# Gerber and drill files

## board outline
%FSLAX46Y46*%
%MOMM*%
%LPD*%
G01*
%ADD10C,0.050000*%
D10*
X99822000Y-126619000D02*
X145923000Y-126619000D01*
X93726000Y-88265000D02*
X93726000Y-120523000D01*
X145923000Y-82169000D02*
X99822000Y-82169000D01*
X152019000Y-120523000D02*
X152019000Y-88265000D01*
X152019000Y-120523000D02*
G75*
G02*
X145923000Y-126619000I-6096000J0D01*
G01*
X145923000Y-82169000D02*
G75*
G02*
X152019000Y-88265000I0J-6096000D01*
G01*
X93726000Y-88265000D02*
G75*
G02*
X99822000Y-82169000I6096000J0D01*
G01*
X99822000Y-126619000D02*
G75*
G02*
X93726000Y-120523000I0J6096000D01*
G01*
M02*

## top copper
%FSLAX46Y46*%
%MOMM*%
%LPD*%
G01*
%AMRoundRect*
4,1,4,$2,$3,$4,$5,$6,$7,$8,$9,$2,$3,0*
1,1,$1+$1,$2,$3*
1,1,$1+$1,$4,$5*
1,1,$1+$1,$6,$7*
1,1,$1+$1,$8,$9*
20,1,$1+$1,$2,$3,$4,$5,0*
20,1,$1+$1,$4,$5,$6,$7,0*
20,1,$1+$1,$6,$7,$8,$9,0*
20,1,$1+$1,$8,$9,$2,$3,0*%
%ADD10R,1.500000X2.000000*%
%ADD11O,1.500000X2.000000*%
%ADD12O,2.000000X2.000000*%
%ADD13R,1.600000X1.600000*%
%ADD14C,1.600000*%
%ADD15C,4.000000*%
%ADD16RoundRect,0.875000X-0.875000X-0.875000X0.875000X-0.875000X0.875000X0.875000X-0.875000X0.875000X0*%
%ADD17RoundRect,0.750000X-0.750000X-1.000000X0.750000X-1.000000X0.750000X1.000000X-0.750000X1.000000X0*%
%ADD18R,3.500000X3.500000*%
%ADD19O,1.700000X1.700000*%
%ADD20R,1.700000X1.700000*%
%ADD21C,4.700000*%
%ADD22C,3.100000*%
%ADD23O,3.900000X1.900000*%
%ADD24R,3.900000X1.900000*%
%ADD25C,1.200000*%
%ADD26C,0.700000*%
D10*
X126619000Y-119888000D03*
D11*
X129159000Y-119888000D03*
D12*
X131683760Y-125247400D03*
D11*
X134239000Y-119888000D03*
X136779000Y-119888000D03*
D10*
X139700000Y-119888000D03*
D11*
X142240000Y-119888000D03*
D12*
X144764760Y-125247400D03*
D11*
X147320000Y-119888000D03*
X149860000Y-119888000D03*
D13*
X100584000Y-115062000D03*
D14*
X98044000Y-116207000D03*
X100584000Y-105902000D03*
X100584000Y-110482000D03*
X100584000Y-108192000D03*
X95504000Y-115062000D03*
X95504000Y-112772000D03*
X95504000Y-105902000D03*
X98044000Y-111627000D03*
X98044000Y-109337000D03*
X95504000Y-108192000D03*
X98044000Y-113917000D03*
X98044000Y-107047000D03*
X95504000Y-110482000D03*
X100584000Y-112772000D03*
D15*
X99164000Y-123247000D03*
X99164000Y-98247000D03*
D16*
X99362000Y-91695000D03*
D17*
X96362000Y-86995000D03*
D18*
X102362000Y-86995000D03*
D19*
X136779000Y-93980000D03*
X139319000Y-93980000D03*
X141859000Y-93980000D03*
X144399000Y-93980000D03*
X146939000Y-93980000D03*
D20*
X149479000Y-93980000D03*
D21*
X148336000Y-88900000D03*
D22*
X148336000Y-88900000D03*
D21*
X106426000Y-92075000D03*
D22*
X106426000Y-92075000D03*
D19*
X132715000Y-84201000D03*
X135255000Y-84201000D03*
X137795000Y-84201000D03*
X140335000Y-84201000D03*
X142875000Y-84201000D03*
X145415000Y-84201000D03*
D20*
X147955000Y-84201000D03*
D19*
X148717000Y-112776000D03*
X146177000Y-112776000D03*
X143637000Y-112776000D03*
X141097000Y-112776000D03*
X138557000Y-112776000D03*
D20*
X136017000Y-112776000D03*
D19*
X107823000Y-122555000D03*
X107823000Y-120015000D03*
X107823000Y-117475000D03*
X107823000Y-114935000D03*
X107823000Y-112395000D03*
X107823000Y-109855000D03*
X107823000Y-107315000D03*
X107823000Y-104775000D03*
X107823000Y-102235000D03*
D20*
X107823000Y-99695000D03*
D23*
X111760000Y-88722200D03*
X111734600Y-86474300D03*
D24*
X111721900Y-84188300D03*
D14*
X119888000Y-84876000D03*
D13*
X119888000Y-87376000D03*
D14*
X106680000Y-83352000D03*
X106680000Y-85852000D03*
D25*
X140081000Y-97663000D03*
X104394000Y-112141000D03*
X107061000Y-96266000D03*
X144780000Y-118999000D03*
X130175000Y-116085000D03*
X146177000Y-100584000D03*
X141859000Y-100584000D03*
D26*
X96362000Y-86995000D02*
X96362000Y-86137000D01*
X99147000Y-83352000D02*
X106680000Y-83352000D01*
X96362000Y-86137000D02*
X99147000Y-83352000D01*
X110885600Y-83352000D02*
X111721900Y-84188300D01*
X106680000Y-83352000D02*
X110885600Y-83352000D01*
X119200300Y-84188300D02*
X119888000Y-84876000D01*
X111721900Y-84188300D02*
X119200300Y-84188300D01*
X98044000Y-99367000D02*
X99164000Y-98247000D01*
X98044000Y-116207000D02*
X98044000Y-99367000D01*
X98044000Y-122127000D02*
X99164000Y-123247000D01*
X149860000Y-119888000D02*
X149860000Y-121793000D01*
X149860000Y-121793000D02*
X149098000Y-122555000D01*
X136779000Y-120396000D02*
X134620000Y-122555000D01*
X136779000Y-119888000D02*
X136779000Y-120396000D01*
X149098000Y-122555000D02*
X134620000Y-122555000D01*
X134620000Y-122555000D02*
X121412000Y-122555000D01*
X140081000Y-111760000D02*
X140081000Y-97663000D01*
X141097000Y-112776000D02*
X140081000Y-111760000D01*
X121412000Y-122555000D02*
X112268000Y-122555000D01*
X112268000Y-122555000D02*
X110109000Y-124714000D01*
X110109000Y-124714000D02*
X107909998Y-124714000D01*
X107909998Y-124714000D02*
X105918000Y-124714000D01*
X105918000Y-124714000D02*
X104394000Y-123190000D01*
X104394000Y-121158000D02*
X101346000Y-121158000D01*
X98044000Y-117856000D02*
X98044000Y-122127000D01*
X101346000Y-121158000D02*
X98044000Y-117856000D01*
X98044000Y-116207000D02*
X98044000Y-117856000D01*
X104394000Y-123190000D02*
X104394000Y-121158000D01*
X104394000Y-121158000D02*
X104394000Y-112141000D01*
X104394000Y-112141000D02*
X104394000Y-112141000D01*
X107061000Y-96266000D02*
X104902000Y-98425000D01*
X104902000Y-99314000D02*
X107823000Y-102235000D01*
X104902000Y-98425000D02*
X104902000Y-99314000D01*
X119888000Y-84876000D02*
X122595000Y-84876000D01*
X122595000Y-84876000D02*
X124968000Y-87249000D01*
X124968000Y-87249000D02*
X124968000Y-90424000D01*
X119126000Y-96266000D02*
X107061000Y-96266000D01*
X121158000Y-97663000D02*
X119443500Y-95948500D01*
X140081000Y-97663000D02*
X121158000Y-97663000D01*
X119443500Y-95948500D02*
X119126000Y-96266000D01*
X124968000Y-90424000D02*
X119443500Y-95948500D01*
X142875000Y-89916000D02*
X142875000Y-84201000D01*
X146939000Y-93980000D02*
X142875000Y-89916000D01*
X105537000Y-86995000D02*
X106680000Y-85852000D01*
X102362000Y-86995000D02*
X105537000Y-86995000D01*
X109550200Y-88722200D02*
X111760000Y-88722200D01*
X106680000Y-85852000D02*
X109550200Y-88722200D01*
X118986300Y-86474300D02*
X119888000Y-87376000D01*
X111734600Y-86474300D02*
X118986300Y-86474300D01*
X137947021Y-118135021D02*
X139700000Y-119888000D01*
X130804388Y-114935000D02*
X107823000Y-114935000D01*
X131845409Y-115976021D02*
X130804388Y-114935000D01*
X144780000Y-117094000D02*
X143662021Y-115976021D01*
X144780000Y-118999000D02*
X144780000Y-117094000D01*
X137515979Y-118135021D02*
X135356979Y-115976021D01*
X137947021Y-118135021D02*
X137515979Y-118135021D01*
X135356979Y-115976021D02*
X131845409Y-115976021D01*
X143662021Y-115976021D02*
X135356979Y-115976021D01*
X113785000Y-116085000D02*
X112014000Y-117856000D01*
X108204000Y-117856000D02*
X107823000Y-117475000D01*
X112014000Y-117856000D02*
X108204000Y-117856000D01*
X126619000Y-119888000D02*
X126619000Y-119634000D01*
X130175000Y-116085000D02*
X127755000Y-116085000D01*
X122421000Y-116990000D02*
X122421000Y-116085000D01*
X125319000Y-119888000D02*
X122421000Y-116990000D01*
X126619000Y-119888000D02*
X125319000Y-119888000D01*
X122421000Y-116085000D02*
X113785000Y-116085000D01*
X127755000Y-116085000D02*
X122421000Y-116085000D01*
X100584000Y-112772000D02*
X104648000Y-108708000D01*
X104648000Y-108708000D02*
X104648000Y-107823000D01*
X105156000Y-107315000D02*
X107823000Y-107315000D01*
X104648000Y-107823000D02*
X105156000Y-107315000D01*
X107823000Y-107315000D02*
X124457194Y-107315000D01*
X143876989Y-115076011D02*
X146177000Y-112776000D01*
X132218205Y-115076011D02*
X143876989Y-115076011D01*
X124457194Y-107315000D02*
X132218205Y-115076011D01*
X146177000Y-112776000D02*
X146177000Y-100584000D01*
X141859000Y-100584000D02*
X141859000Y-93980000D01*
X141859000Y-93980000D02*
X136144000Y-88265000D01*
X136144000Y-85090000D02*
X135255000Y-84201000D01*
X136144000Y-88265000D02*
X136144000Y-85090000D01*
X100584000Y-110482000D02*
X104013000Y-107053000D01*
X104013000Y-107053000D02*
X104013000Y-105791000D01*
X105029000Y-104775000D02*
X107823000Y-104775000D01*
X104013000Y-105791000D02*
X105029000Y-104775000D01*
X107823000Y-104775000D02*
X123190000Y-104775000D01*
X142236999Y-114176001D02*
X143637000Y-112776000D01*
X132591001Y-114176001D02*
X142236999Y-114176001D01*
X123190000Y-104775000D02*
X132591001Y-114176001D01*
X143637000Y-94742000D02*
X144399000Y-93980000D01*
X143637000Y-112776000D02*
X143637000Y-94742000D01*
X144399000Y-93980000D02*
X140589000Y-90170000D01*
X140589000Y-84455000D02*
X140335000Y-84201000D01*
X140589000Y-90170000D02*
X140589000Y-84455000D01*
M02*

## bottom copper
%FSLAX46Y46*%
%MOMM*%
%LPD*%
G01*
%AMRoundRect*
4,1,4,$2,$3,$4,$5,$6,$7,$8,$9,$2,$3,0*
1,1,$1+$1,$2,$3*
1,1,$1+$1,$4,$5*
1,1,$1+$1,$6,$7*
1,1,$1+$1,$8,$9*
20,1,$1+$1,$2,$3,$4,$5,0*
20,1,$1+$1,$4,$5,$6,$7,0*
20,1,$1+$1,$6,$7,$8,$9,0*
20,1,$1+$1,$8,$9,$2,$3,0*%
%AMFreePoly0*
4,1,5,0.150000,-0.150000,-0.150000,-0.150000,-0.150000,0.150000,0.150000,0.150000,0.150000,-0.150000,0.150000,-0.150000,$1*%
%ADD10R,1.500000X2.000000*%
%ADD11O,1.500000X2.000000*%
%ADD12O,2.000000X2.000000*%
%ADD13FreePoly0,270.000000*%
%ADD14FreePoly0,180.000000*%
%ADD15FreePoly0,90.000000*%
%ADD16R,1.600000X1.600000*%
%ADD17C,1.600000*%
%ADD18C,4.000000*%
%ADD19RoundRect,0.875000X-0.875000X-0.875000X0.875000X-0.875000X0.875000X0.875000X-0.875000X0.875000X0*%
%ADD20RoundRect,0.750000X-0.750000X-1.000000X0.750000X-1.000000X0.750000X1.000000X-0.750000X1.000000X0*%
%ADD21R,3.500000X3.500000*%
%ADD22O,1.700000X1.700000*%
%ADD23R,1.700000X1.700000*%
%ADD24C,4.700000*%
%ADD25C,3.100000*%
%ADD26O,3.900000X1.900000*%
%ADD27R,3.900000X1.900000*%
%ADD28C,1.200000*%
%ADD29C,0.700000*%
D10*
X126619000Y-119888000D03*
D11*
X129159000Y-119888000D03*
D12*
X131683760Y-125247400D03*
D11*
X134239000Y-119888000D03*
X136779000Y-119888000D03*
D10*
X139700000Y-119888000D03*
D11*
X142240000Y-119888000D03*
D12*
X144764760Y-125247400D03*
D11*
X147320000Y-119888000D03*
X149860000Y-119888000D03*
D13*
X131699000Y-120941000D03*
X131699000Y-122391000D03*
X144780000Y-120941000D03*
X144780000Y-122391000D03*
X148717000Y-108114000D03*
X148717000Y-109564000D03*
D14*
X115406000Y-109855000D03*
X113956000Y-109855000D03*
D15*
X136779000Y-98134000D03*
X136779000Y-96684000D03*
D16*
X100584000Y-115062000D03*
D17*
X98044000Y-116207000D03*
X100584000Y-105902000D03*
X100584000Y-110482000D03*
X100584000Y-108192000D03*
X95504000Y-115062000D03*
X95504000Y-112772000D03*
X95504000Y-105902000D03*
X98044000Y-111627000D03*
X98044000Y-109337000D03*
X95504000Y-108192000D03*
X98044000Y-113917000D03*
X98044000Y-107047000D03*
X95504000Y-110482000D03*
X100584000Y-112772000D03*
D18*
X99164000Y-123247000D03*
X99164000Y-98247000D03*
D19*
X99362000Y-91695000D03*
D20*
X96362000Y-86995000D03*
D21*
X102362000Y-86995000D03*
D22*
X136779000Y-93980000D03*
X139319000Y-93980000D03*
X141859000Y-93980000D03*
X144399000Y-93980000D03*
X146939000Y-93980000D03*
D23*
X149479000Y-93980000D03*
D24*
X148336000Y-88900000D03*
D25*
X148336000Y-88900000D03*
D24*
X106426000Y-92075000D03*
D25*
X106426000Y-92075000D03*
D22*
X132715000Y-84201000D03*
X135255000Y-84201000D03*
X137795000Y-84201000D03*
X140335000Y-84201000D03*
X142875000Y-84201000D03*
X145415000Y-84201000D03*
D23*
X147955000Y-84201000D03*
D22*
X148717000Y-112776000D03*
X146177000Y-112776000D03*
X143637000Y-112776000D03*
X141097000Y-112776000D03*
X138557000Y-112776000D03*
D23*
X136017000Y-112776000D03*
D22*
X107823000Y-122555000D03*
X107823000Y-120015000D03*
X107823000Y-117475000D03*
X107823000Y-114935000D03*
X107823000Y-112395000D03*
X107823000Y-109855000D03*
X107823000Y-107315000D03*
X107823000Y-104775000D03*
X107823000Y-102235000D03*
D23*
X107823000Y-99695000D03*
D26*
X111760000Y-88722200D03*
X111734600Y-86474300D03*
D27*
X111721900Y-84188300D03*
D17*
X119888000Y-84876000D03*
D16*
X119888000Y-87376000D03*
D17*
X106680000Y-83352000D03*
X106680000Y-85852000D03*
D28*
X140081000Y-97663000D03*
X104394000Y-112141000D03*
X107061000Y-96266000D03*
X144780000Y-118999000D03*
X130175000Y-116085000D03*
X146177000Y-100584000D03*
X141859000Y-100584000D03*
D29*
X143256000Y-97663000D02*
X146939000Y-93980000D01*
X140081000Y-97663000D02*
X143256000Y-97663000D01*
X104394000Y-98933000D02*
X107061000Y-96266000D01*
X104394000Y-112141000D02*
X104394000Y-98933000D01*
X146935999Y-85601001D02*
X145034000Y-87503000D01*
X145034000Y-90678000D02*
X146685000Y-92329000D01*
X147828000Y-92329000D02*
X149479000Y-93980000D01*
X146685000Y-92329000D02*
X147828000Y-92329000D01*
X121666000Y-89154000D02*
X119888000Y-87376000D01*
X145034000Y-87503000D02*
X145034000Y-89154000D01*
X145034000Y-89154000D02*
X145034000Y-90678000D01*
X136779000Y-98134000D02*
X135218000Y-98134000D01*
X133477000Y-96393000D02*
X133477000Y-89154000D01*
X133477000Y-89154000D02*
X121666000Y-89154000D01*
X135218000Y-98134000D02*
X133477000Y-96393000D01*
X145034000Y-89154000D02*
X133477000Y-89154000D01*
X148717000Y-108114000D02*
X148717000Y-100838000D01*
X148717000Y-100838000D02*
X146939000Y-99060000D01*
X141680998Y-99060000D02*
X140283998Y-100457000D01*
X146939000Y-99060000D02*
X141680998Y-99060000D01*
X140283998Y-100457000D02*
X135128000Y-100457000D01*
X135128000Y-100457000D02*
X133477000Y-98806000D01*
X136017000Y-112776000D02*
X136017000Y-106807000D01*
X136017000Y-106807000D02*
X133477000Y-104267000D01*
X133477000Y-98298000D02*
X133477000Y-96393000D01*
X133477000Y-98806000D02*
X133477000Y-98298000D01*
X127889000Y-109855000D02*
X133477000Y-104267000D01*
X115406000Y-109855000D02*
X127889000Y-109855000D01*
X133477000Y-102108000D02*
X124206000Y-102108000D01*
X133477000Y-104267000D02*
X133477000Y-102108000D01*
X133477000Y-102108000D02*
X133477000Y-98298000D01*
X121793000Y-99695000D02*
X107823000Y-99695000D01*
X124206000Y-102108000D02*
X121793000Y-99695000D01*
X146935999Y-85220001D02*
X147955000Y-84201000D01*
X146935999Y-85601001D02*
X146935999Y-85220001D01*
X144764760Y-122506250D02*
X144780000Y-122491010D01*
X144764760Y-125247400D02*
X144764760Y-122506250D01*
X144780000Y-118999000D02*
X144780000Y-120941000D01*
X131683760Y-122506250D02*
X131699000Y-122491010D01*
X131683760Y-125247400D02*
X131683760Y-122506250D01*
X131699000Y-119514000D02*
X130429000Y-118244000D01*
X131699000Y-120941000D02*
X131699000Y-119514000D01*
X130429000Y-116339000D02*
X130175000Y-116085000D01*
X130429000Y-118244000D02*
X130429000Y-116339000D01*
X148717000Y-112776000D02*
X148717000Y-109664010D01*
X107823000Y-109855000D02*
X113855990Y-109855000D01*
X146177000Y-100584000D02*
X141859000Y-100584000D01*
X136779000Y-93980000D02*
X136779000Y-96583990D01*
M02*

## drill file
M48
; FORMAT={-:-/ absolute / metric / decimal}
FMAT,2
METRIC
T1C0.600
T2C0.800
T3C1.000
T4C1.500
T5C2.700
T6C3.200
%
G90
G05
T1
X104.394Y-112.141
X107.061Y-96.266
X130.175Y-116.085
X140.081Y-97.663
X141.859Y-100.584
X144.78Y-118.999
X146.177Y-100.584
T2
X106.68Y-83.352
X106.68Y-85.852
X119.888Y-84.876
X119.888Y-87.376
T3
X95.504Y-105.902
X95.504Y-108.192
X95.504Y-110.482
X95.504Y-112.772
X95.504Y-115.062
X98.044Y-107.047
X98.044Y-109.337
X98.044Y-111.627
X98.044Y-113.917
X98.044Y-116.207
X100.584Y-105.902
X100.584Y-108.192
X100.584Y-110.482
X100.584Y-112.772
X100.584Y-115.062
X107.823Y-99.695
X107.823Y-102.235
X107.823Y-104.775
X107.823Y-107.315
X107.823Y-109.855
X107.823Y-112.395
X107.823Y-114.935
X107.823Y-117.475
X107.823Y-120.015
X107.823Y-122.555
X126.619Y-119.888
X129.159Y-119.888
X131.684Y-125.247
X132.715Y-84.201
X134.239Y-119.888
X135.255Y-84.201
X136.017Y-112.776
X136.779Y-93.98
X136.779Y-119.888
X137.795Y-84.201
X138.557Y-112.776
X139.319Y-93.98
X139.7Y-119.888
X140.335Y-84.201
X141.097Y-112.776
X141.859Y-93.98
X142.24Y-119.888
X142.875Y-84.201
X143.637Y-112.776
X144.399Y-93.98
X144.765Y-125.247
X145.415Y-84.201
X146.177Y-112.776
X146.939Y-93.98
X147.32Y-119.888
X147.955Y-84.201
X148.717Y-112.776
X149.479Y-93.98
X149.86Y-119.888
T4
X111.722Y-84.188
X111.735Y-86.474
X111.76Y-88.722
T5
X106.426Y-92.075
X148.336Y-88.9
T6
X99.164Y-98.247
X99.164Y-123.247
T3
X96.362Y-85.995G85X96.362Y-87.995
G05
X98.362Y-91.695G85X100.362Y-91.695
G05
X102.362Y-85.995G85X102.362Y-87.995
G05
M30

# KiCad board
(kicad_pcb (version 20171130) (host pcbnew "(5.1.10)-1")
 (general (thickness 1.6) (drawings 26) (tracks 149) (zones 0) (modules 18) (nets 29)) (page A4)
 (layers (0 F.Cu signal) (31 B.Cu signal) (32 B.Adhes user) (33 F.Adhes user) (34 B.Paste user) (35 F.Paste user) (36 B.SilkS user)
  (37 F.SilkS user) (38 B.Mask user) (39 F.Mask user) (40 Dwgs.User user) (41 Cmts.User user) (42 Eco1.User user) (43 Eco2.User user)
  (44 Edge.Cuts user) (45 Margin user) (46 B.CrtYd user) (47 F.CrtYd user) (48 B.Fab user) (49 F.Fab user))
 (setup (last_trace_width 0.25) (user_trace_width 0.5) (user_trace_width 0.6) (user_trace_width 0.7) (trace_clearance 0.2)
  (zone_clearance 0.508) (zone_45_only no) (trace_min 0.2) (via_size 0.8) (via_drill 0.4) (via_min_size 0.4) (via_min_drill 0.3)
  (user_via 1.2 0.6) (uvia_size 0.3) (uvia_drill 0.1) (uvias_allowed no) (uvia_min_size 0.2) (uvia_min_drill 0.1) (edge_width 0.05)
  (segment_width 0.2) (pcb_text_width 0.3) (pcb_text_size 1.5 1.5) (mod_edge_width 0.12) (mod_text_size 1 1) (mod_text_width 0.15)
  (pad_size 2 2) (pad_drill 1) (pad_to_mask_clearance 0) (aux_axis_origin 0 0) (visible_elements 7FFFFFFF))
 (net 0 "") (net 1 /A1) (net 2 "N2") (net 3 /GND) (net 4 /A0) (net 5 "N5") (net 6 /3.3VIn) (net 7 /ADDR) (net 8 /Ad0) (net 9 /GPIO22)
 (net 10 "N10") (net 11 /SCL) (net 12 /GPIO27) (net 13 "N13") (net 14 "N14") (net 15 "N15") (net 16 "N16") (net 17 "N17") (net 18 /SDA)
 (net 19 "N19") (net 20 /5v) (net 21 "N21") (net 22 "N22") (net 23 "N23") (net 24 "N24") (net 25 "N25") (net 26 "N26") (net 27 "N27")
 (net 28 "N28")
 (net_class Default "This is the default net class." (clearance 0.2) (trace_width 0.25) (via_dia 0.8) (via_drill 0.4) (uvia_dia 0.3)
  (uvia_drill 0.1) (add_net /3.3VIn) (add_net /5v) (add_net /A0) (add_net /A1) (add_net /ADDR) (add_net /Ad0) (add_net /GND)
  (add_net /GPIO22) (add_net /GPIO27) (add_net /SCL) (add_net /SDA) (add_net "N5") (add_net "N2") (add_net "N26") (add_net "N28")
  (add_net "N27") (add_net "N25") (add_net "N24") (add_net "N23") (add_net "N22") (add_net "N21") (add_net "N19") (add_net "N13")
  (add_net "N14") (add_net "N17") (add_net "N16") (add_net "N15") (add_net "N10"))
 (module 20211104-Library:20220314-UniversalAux (layer F.Cu) (at 131.699 121.158 180)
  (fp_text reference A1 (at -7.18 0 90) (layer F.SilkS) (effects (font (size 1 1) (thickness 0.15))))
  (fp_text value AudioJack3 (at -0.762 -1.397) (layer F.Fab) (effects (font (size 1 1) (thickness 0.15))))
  (pad S thru_hole rect (at 5.08 1.27 180) (size 1.5 2) (drill 1) (layers *.Cu *.Mask) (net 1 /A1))
  (pad "" thru_hole oval (at 2.54 1.27 180) (size 1.5 2) (drill 1) (layers *.Cu *.Mask))
  (pad R thru_hole oval (at 0.01524 -4.0894 180) (size 2 2) (drill 1) (layers *.Cu *.Mask) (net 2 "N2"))
  (pad "" thru_hole oval (at -2.54 1.27 180) (size 1.5 2) (drill 1) (layers *.Cu *.Mask))
  (pad T thru_hole oval (at -5.08 1.27 180) (size 1.5 2) (drill 1) (layers *.Cu *.Mask) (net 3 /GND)))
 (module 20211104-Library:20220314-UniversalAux (layer F.Cu) (at 144.78 121.158 180)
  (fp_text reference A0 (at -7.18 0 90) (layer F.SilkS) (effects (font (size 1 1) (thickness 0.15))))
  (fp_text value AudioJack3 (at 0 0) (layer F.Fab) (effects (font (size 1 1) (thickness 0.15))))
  (pad S thru_hole rect (at 5.08 1.27 180) (size 1.5 2) (drill 1) (layers *.Cu *.Mask) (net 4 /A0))
  (pad "" thru_hole oval (at 2.54 1.27 180) (size 1.5 2) (drill 1) (layers *.Cu *.Mask))
  (pad R thru_hole oval (at 0.01524 -4.0894 180) (size 2 2) (drill 1) (layers *.Cu *.Mask) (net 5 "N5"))
  (pad "" thru_hole oval (at -2.54 1.27 180) (size 1.5 2) (drill 1) (layers *.Cu *.Mask))
  (pad T thru_hole oval (at -5.08 1.27 180) (size 1.5 2) (drill 1) (layers *.Cu *.Mask) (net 3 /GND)))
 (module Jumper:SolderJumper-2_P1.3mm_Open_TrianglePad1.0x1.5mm (layer B.Cu) (at 131.699 121.666 270)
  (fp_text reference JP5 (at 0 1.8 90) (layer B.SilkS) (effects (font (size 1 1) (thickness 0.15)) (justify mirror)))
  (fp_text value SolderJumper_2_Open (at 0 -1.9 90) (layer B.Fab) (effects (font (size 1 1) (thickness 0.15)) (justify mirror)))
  (pad 1 smd custom (at -0.725 0 270) (size 0.3 0.3) (layers B.Cu B.Mask) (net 1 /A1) (zone_connect 2)
   (options (clearance outline) (anchor rect)) (primitives))
  (pad 2 smd custom (at 0.725 0 270) (size 0.3 0.3) (layers B.Cu B.Mask) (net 2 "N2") (zone_connect 2)
   (options (clearance outline) (anchor rect)) (primitives)))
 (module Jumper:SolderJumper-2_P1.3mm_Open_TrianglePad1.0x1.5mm (layer B.Cu) (at 144.78 121.666 270)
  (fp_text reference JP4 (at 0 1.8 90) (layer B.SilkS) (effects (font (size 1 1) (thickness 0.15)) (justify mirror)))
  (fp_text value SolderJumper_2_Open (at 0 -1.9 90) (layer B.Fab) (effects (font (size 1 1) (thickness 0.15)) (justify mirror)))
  (pad 1 smd custom (at -0.725 0 270) (size 0.3 0.3) (layers B.Cu B.Mask) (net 4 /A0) (zone_connect 2)
   (options (clearance outline) (anchor rect)) (primitives))
  (pad 2 smd custom (at 0.725 0 270) (size 0.3 0.3) (layers B.Cu B.Mask) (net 5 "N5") (zone_connect 2)
   (options (clearance outline) (anchor rect)) (primitives)))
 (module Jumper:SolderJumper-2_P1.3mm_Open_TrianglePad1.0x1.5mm (layer B.Cu) (at 148.717 108.839 270)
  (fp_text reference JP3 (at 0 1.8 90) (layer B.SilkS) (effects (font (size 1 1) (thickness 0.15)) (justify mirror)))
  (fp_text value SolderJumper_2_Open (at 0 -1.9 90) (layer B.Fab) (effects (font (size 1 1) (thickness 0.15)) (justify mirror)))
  (pad 1 smd custom (at -0.725 0 270) (size 0.3 0.3) (layers B.Cu B.Mask) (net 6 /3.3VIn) (zone_connect 2)
   (options (clearance outline) (anchor rect)) (primitives))
  (pad 2 smd custom (at 0.725 0 270) (size 0.3 0.3) (layers B.Cu B.Mask) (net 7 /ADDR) (zone_connect 2)
   (options (clearance outline) (anchor rect)) (primitives)))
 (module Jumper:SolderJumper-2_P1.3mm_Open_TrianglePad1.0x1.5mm (layer B.Cu) (at 114.681 109.855 180)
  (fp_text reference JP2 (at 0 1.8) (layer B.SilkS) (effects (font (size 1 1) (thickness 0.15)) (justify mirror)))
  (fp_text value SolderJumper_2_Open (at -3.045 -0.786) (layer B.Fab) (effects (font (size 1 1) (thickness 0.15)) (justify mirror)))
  (pad 1 smd custom (at -0.725 0 180) (size 0.3 0.3) (layers B.Cu B.Mask) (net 6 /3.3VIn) (zone_connect 2)
   (options (clearance outline) (anchor rect)) (primitives))
  (pad 2 smd custom (at 0.725 0 180) (size 0.3 0.3) (layers B.Cu B.Mask) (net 7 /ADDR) (zone_connect 2)
   (options (clearance outline) (anchor rect)) (primitives)))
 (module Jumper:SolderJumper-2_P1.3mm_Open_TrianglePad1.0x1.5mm (layer B.Cu) (at 136.779 97.409 90)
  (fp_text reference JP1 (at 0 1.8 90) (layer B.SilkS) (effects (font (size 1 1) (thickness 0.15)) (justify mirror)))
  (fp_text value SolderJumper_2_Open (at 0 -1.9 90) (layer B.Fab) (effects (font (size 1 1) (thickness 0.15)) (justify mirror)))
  (pad 1 smd custom (at -0.725 0 90) (size 0.3 0.3) (layers B.Cu B.Mask) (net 6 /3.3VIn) (zone_connect 2)
   (options (clearance outline) (anchor rect)) (primitives))
  (pad 2 smd custom (at 0.725 0 90) (size 0.3 0.3) (layers B.Cu B.Mask) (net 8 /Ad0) (zone_connect 2)
   (options (clearance outline) (anchor rect)) (primitives)))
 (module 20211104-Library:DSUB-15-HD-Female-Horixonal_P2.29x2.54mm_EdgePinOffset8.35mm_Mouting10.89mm (layer F.Cu) (at 100.584 115.062 270)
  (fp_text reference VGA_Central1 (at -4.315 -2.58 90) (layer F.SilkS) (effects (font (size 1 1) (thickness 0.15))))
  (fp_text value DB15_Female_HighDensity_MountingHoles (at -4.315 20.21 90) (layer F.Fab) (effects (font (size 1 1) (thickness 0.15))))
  (pad 1 thru_hole rect (at 0 0 270) (size 1.6 1.6) (drill 1) (layers *.Cu *.Mask) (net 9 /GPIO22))
  (pad 6 thru_hole circle (at 1.145 2.54 270) (size 1.6 1.6) (drill 1) (layers *.Cu *.Mask) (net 3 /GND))
  (pad 5 thru_hole circle (at -9.16 0 270) (size 1.6 1.6) (drill 1) (layers *.Cu *.Mask) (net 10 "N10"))
  (pad 3 thru_hole circle (at -4.58 0 270) (size 1.6 1.6) (drill 1) (layers *.Cu *.Mask) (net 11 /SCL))
  (pad 4 thru_hole circle (at -6.87 0 270) (size 1.6 1.6) (drill 1) (layers *.Cu *.Mask) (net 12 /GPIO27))
  (pad 11 thru_hole circle (at 0 5.08 270) (size 1.6 1.6) (drill 1) (layers *.Cu *.Mask) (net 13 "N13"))
  (pad 12 thru_hole circle (at -2.29 5.08 270) (size 1.6 1.6) (drill 1) (layers *.Cu *.Mask) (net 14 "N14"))
  (pad 15 thru_hole circle (at -9.16 5.08 270) (size 1.6 1.6) (drill 1) (layers *.Cu *.Mask) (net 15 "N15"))
  (pad 8 thru_hole circle (at -3.435 2.54 270) (size 1.6 1.6) (drill 1) (layers *.Cu *.Mask) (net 3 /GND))
  (pad 9 thru_hole circle (at -5.725 2.54 270) (size 1.6 1.6) (drill 1) (layers *.Cu *.Mask) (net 3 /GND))
  (pad 14 thru_hole circle (at -6.87 5.08 270) (size 1.6 1.6) (drill 1) (layers *.Cu *.Mask) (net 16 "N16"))
  (pad 7 thru_hole circle (at -1.145 2.54 270) (size 1.6 1.6) (drill 1) (layers *.Cu *.Mask) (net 3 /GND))
  (pad 10 thru_hole circle (at -8.015 2.54 270) (size 1.6 1.6) (drill 1) (layers *.Cu *.Mask) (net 3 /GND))
  (pad 13 thru_hole circle (at -4.58 5.08 270) (size 1.6 1.6) (drill 1) (layers *.Cu *.Mask) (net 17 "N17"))
  (pad 2 thru_hole circle (at -2.29 0 270) (size 1.6 1.6) (drill 1) (layers *.Cu *.Mask) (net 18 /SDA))
  (pad 0 thru_hole circle (at 8.185 1.42 270) (size 4 4) (drill 3.2) (layers *.Cu *.Mask) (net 3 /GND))
  (pad 0 thru_hole circle (at -16.815 1.42 270) (size 4 4) (drill 3.2) (layers *.Cu *.Mask) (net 3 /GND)))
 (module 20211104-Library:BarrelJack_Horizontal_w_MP (layer F.Cu) (at 102.362 86.995)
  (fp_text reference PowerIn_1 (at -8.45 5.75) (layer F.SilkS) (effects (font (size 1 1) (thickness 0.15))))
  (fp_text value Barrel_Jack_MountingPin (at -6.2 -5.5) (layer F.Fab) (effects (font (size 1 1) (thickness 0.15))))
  (pad MP thru_hole roundrect (at -3 4.7) (size 3.5 3.5) (drill oval 3 1) (layers *.Cu *.Mask) (roundrect_rratio 0.25) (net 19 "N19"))
  (pad 2 thru_hole roundrect (at -6 0) (size 3 3.5) (drill oval 1 3) (layers *.Cu *.Mask) (roundrect_rratio 0.25) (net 3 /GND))
  (pad 1 thru_hole rect (at 0 0) (size 3.5 3.5) (drill oval 1 3) (layers *.Cu *.Mask) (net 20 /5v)))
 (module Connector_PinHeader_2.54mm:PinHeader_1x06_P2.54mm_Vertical (layer F.Cu) (at 149.479 93.98 270)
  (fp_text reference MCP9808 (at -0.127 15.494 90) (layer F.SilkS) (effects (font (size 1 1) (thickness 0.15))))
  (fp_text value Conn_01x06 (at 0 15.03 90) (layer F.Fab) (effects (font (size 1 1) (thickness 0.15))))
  (pad 6 thru_hole oval (at 0 12.7 270) (size 1.7 1.7) (drill 1) (layers *.Cu *.Mask) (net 8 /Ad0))
  (pad 5 thru_hole oval (at 0 10.16 270) (size 1.7 1.7) (drill 1) (layers *.Cu *.Mask) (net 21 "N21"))
  (pad 4 thru_hole oval (at 0 7.62 270) (size 1.7 1.7) (drill 1) (layers *.Cu *.Mask) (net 18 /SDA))
  (pad 3 thru_hole oval (at 0 5.08 270) (size 1.7 1.7) (drill 1) (layers *.Cu *.Mask) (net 11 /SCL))
  (pad 2 thru_hole oval (at 0 2.54 270) (size 1.7 1.7) (drill 1) (layers *.Cu *.Mask) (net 3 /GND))
  (pad 1 thru_hole rect (at 0 0 270) (size 1.7 1.7) (drill 1) (layers *.Cu *.Mask) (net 6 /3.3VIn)))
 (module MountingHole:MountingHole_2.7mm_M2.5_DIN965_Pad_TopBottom (layer F.Cu) (at 148.336 88.9)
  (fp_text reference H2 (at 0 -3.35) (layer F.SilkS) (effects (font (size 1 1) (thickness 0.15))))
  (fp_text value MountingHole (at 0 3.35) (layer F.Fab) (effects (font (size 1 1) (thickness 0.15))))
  (pad 1 connect circle (at 0 0) (size 4.7 4.7) (layers B.Cu B.Mask))
  (pad 1 connect circle (at 0 0) (size 4.7 4.7) (layers F.Cu F.Mask))
  (pad 1 thru_hole circle (at 0 0) (size 3.1 3.1) (drill 2.7) (layers *.Cu *.Mask)))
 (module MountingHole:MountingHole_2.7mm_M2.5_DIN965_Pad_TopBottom (layer F.Cu) (at 106.426 92.075)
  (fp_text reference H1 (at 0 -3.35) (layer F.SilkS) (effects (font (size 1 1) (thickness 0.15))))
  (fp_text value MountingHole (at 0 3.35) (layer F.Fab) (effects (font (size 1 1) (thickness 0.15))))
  (pad 1 connect circle (at 0 0) (size 4.7 4.7) (layers B.Cu B.Mask))
  (pad 1 connect circle (at 0 0) (size 4.7 4.7) (layers F.Cu F.Mask))
  (pad 1 thru_hole circle (at 0 0) (size 3.1 3.1) (drill 2.7) (layers *.Cu *.Mask)))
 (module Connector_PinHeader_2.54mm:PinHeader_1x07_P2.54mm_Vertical (layer F.Cu) (at 147.955 84.201 270)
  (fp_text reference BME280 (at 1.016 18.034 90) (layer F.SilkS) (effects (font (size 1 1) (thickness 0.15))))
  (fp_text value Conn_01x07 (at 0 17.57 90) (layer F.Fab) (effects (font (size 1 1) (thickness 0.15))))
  (pad 7 thru_hole oval (at 0 15.24 270) (size 1.7 1.7) (drill 1) (layers *.Cu *.Mask) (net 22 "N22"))
  (pad 6 thru_hole oval (at 0 12.7 270) (size 1.7 1.7) (drill 1) (layers *.Cu *.Mask) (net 18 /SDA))
  (pad 5 thru_hole oval (at 0 10.16 270) (size 1.7 1.7) (drill 1) (layers *.Cu *.Mask) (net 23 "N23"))
  (pad 4 thru_hole oval (at 0 7.62 270) (size 1.7 1.7) (drill 1) (layers *.Cu *.Mask) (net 11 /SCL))
  (pad 3 thru_hole oval (at 0 5.08 270) (size 1.7 1.7) (drill 1) (layers *.Cu *.Mask) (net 3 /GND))
  (pad 2 thru_hole oval (at 0 2.54 270) (size 1.7 1.7) (drill 1) (layers *.Cu *.Mask) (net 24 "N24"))
  (pad 1 thru_hole rect (at 0 0 270) (size 1.7 1.7) (drill 1) (layers *.Cu *.Mask) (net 6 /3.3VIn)))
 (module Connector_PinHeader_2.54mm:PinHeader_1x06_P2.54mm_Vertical (layer F.Cu) (at 136.017 112.776 90)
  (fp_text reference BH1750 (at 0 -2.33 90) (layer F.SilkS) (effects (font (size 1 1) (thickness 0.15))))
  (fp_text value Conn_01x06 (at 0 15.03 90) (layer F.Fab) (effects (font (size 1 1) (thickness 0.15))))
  (pad 6 thru_hole oval (at 0 12.7 90) (size 1.7 1.7) (drill 1) (layers *.Cu *.Mask) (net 7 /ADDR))
  (pad 5 thru_hole oval (at 0 10.16 90) (size 1.7 1.7) (drill 1) (layers *.Cu *.Mask) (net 18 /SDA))
  (pad 4 thru_hole oval (at 0 7.62 90) (size 1.7 1.7) (drill 1) (layers *.Cu *.Mask) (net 11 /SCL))
  (pad 3 thru_hole oval (at 0 5.08 90) (size 1.7 1.7) (drill 1) (layers *.Cu *.Mask) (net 3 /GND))
  (pad 2 thru_hole oval (at 0 2.54 90) (size 1.7 1.7) (drill 1) (layers *.Cu *.Mask) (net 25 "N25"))
  (pad 1 thru_hole rect (at 0 0 90) (size 1.7 1.7) (drill 1) (layers *.Cu *.Mask) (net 6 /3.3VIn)))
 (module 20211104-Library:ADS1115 (layer F.Cu) (at 107.823 99.695)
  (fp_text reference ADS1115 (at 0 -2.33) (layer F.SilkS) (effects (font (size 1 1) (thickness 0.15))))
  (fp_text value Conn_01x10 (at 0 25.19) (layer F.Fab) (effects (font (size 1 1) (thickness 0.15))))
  (pad 10 thru_hole oval (at 0 22.86) (size 1.7 1.7) (drill 1) (layers *.Cu *.Mask) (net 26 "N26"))
  (pad 9 thru_hole oval (at 0 20.32) (size 1.7 1.7) (drill 1) (layers *.Cu *.Mask) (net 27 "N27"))
  (pad 8 thru_hole oval (at 0 17.78) (size 1.7 1.7) (drill 1) (layers *.Cu *.Mask) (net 1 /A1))
  (pad 7 thru_hole oval (at 0 15.24) (size 1.7 1.7) (drill 1) (layers *.Cu *.Mask) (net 4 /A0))
  (pad 6 thru_hole oval (at 0 12.7) (size 1.7 1.7) (drill 1) (layers *.Cu *.Mask) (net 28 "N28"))
  (pad 5 thru_hole oval (at 0 10.16) (size 1.7 1.7) (drill 1) (layers *.Cu *.Mask) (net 7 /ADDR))
  (pad 4 thru_hole oval (at 0 7.62) (size 1.7 1.7) (drill 1) (layers *.Cu *.Mask) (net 18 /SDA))
  (pad 3 thru_hole oval (at 0 5.08) (size 1.7 1.7) (drill 1) (layers *.Cu *.Mask) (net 11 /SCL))
  (pad 2 thru_hole oval (at 0 2.54) (size 1.7 1.7) (drill 1) (layers *.Cu *.Mask) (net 3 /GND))
  (pad 1 thru_hole rect (at 0 0) (size 1.7 1.7) (drill 1) (layers *.Cu *.Mask) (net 6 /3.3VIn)))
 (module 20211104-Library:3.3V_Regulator (layer F.Cu) (at 111.76 81.026 270)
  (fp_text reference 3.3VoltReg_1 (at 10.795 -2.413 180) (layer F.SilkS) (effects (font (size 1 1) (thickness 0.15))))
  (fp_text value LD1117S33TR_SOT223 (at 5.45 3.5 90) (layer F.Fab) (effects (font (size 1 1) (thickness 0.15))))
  (pad 3 thru_hole oval (at 7.6962 0 270) (size 1.9 3.9) (drill 1.5) (layers *.Cu *.Mask) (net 20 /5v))
  (pad 2 thru_hole oval (at 5.4483 0.0254 270) (size 1.9 3.9) (drill 1.5) (layers *.Cu *.Mask) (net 6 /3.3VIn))
  (pad 1 thru_hole rect (at 3.1623 0.0381 270) (size 1.9 3.9) (drill 1.5) (layers *.Cu *.Mask) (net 3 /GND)))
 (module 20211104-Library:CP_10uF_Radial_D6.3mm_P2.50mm (layer F.Cu) (at 119.888 87.376 90)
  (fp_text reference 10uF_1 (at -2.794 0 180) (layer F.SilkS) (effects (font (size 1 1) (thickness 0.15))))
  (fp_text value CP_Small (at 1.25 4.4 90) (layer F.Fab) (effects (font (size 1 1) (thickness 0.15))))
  (pad 2 thru_hole circle (at 2.5 0 90) (size 1.6 1.6) (drill 0.8) (layers *.Cu *.Mask) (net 3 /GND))
  (pad 1 thru_hole rect (at 0 0 90) (size 1.6 1.6) (drill 0.8) (layers *.Cu *.Mask) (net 6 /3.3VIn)))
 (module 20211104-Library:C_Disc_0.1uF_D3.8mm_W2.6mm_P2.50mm (layer F.Cu) (at 106.68 85.852 90)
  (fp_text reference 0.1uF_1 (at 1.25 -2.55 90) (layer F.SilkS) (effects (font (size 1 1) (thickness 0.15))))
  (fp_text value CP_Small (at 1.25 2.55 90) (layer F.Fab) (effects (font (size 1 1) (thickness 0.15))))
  (pad 2 thru_hole circle (at 2.5 0 90) (size 1.6 1.6) (drill 0.8) (layers *.Cu *.Mask) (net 3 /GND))
  (pad 1 thru_hole circle (at 0 0 90) (size 1.6 1.6) (drill 0.8) (layers *.Cu *.Mask) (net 20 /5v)))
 (gr_line (start 99.822 126.619) (end 145.923 126.619) (layer Edge.Cuts) (width 0.05))
 (gr_line (start 93.726 88.265) (end 93.726 120.523) (layer Edge.Cuts) (width 0.05))
 (gr_line (start 145.923 82.169) (end 99.822 82.169) (layer Edge.Cuts) (width 0.05))
 (gr_line (start 152.019 120.523) (end 152.019 88.265) (layer Edge.Cuts) (width 0.05))
 (gr_arc (start 145.923 120.523) (end 145.923 126.619) (angle -90) (layer Edge.Cuts) (width 0.05))
 (gr_arc (start 145.923 88.265) (end 152.019 88.265) (angle -90) (layer Edge.Cuts) (width 0.05))
 (gr_arc (start 99.822 88.265) (end 99.822 82.169) (angle -90) (layer Edge.Cuts) (width 0.05))
 (gr_arc (start 99.822 120.523) (end 93.726 120.523) (angle -90) (layer Edge.Cuts) (width 0.05))
 (segment (start 96.362 86.995) (end 96.362 86.137) (width 0.7) (layer F.Cu) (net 3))
 (segment (start 99.147 83.352) (end 106.68 83.352) (width 0.7) (layer F.Cu) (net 3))
 (segment (start 96.362 86.137) (end 99.147 83.352) (width 0.7) (layer F.Cu) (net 3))
 (segment (start 110.8856 83.352) (end 111.7219 84.1883) (width 0.7) (layer F.Cu) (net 3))
 (segment (start 106.68 83.352) (end 110.8856 83.352) (width 0.7) (layer F.Cu) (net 3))
 (segment (start 119.2003 84.1883) (end 119.888 84.876) (width 0.7) (layer F.Cu) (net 3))
 (segment (start 111.7219 84.1883) (end 119.2003 84.1883) (width 0.7) (layer F.Cu) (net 3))
 (segment (start 98.044 99.367) (end 99.164 98.247) (width 0.7) (layer F.Cu) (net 3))
 (segment (start 98.044 116.207) (end 98.044 99.367) (width 0.7) (layer F.Cu) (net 3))
 (segment (start 98.044 122.127) (end 99.164 123.247) (width 0.7) (layer F.Cu) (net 3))
 (segment (start 149.86 119.888) (end 149.86 121.793) (width 0.7) (layer F.Cu) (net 3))
 (segment (start 149.86 121.793) (end 149.098 122.555) (width 0.7) (layer F.Cu) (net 3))
 (segment (start 136.779 120.396) (end 134.62 122.555) (width 0.7) (layer F.Cu) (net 3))
 (segment (start 136.779 119.888) (end 136.779 120.396) (width 0.7) (layer F.Cu) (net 3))
 (segment (start 149.098 122.555) (end 134.62 122.555) (width 0.7) (layer F.Cu) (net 3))
 (segment (start 134.62 122.555) (end 121.412 122.555) (width 0.7) (layer F.Cu) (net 3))
 (via (at 140.081 97.663) (size 1.2) (drill 0.6) (layers F.Cu B.Cu) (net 3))
 (segment (start 140.081 111.76) (end 140.081 97.663) (width 0.7) (layer F.Cu) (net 3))
 (segment (start 141.097 112.776) (end 140.081 111.76) (width 0.7) (layer F.Cu) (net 3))
 (segment (start 143.256 97.663) (end 146.939 93.98) (width 0.7) (layer B.Cu) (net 3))
 (segment (start 140.081 97.663) (end 143.256 97.663) (width 0.7) (layer B.Cu) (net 3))
 (segment (start 121.412 122.555) (end 112.268 122.555) (width 0.7) (layer F.Cu) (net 3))
 (segment (start 112.268 122.555) (end 110.109 124.714) (width 0.7) (layer F.Cu) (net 3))
 (segment (start 110.109 124.714) (end 107.909998 124.714) (width 0.7) (layer F.Cu) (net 3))
 (segment (start 107.909998 124.714) (end 105.918 124.714) (width 0.7) (layer F.Cu) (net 3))
 (segment (start 105.918 124.714) (end 104.394 123.19) (width 0.7) (layer F.Cu) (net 3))
 (segment (start 104.394 121.158) (end 101.346 121.158) (width 0.7) (layer F.Cu) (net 3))
 (segment (start 98.044 117.856) (end 98.044 122.127) (width 0.7) (layer F.Cu) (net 3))
 (segment (start 101.346 121.158) (end 98.044 117.856) (width 0.7) (layer F.Cu) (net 3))
 (segment (start 98.044 116.207) (end 98.044 117.856) (width 0.7) (layer F.Cu) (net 3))
 (segment (start 104.394 123.19) (end 104.394 121.158) (width 0.7) (layer F.Cu) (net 3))
 (segment (start 104.394 121.158) (end 104.394 112.141) (width 0.7) (layer F.Cu) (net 3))
 (segment (start 104.394 112.141) (end 104.394 112.141) (width 0.7) (layer F.Cu) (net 3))
 (via (at 104.394 112.141) (size 1.2) (drill 0.6) (layers F.Cu B.Cu) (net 3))
 (via (at 107.061 96.266) (size 1.2) (drill 0.6) (layers F.Cu B.Cu) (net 3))
 (segment (start 104.394 98.933) (end 107.061 96.266) (width 0.7) (layer B.Cu) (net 3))
 (segment (start 104.394 112.141) (end 104.394 98.933) (width 0.7) (layer B.Cu) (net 3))
 (segment (start 107.061 96.266) (end 104.902 98.425) (width 0.7) (layer F.Cu) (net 3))
 (segment (start 104.902 99.314) (end 107.823 102.235) (width 0.7) (layer F.Cu) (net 3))
 (segment (start 104.902 98.425) (end 104.902 99.314) (width 0.7) (layer F.Cu) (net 3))
 (segment (start 119.888 84.876) (end 122.595 84.876) (width 0.7) (layer F.Cu) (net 3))
 (segment (start 122.595 84.876) (end 124.968 87.249) (width 0.7) (layer F.Cu) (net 3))
 (segment (start 124.968 87.249) (end 124.968 90.424) (width 0.7) (layer F.Cu) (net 3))
 (segment (start 119.126 96.266) (end 107.061 96.266) (width 0.7) (layer F.Cu) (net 3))
 (segment (start 121.158 97.663) (end 119.4435 95.9485) (width 0.7) (layer F.Cu) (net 3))
 (segment (start 140.081 97.663) (end 121.158 97.663) (width 0.7) (layer F.Cu) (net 3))
 (segment (start 119.4435 95.9485) (end 119.126 96.266) (width 0.7) (layer F.Cu) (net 3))
 (segment (start 124.968 90.424) (end 119.4435 95.9485) (width 0.7) (layer F.Cu) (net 3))
 (segment (start 142.875 89.916) (end 142.875 84.201) (width 0.7) (layer F.Cu) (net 3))
 (segment (start 146.939 93.98) (end 142.875 89.916) (width 0.7) (layer F.Cu) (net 3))
 (segment (start 105.537 86.995) (end 106.68 85.852) (width 0.7) (layer F.Cu) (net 20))
 (segment (start 102.362 86.995) (end 105.537 86.995) (width 0.7) (layer F.Cu) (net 20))
 (segment (start 109.5502 88.7222) (end 111.76 88.7222) (width 0.7) (layer F.Cu) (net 20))
 (segment (start 106.68 85.852) (end 109.5502 88.7222) (width 0.7) (layer F.Cu) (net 20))
 (segment (start 118.9863 86.4743) (end 119.888 87.376) (width 0.7) (layer F.Cu) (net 6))
 (segment (start 111.7346 86.4743) (end 118.9863 86.4743) (width 0.7) (layer F.Cu) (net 6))
 (segment (start 146.935999 85.601001) (end 145.034 87.503) (width 0.7) (layer B.Cu) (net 6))
 (segment (start 145.034 90.678) (end 146.685 92.329) (width 0.7) (layer B.Cu) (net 6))
 (segment (start 147.828 92.329) (end 149.479 93.98) (width 0.7) (layer B.Cu) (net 6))
 (segment (start 146.685 92.329) (end 147.828 92.329) (width 0.7) (layer B.Cu) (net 6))
 (segment (start 121.666 89.154) (end 119.888 87.376) (width 0.7) (layer B.Cu) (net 6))
 (segment (start 145.034 87.503) (end 145.034 89.154) (width 0.7) (layer B.Cu) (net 6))
 (segment (start 145.034 89.154) (end 145.034 90.678) (width 0.7) (layer B.Cu) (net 6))
 (segment (start 136.779 98.134) (end 135.218 98.134) (width 0.7) (layer B.Cu) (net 6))
 (segment (start 133.477 96.393) (end 133.477 89.154) (width 0.7) (layer B.Cu) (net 6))
 (segment (start 133.477 89.154) (end 121.666 89.154) (width 0.7) (layer B.Cu) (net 6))
 (segment (start 135.218 98.134) (end 133.477 96.393) (width 0.7) (layer B.Cu) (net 6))
 (segment (start 145.034 89.154) (end 133.477 89.154) (width 0.7) (layer B.Cu) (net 6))
 (segment (start 148.717 108.114) (end 148.717 100.838) (width 0.7) (layer B.Cu) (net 6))
 (segment (start 148.717 100.838) (end 146.939 99.06) (width 0.7) (layer B.Cu) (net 6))
 (segment (start 141.680998 99.06) (end 140.283998 100.457) (width 0.7) (layer B.Cu) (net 6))
 (segment (start 146.939 99.06) (end 141.680998 99.06) (width 0.7) (layer B.Cu) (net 6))
 (segment (start 140.283998 100.457) (end 135.128 100.457) (width 0.7) (layer B.Cu) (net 6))
 (segment (start 135.128 100.457) (end 133.477 98.806) (width 0.7) (layer B.Cu) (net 6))
 (segment (start 136.017 112.776) (end 136.017 106.807) (width 0.7) (layer B.Cu) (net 6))
 (segment (start 136.017 106.807) (end 133.477 104.267) (width 0.7) (layer B.Cu) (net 6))
 (segment (start 133.477 98.298) (end 133.477 96.393) (width 0.7) (layer B.Cu) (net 6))
 (segment (start 133.477 98.806) (end 133.477 98.298) (width 0.7) (layer B.Cu) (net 6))
 (segment (start 127.889 109.855) (end 133.477 104.267) (width 0.7) (layer B.Cu) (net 6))
 (segment (start 115.406 109.855) (end 127.889 109.855) (width 0.7) (layer B.Cu) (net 6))
 (segment (start 133.477 102.108) (end 124.206 102.108) (width 0.7) (layer B.Cu) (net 6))
 (segment (start 133.477 104.267) (end 133.477 102.108) (width 0.7) (layer B.Cu) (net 6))
 (segment (start 133.477 102.108) (end 133.477 98.298) (width 0.7) (layer B.Cu) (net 6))
 (segment (start 121.793 99.695) (end 107.823 99.695) (width 0.7) (layer B.Cu) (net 6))
 (segment (start 124.206 102.108) (end 121.793 99.695) (width 0.7) (layer B.Cu) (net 6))
 (segment (start 146.935999 85.220001) (end 147.955 84.201) (width 0.7) (layer B.Cu) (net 6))
 (segment (start 146.935999 85.601001) (end 146.935999 85.220001) (width 0.7) (layer B.Cu) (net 6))
 (segment (start 144.76476 122.50625) (end 144.78 122.49101) (width 0.7) (layer B.Cu) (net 5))
 (segment (start 144.76476 125.2474) (end 144.76476 122.50625) (width 0.7) (layer B.Cu) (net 5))
 (segment (start 137.947021 118.135021) (end 139.7 119.888) (width 0.7) (layer F.Cu) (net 4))
 (via (at 144.78 118.999) (size 1.2) (drill 0.6) (layers F.Cu B.Cu) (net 4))
 (segment (start 144.78 118.999) (end 144.78 120.941) (width 0.7) (layer B.Cu) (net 4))
 (segment (start 130.804388 114.935) (end 107.823 114.935) (width 0.7) (layer F.Cu) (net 4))
 (segment (start 131.845409 115.976021) (end 130.804388 114.935) (width 0.7) (layer F.Cu) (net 4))
 (segment (start 144.78 117.094) (end 143.662021 115.976021) (width 0.7) (layer F.Cu) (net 4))
 (segment (start 144.78 118.999) (end 144.78 117.094) (width 0.7) (layer F.Cu) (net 4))
 (segment (start 137.515979 118.135021) (end 135.356979 115.976021) (width 0.7) (layer F.Cu) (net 4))
 (segment (start 137.947021 118.135021) (end 137.515979 118.135021) (width 0.7) (layer F.Cu) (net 4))
 (segment (start 135.356979 115.976021) (end 131.845409 115.976021) (width 0.7) (layer F.Cu) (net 4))
 (segment (start 143.662021 115.976021) (end 135.356979 115.976021) (width 0.7) (layer F.Cu) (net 4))
 (segment (start 131.68376 122.50625) (end 131.699 122.49101) (width 0.7) (layer B.Cu) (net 2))
 (segment (start 131.68376 125.2474) (end 131.68376 122.50625) (width 0.7) (layer B.Cu) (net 2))
 (via (at 130.175 116.085) (size 1.2) (drill 0.6) (layers F.Cu B.Cu) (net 1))
 (segment (start 131.699 119.514) (end 130.429 118.244) (width 0.7) (layer B.Cu) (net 1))
 (segment (start 131.699 120.941) (end 131.699 119.514) (width 0.7) (layer B.Cu) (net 1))
 (segment (start 113.785 116.085) (end 112.014 117.856) (width 0.7) (layer F.Cu) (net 1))
 (segment (start 108.204 117.856) (end 107.823 117.475) (width 0.7) (layer F.Cu) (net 1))
 (segment (start 112.014 117.856) (end 108.204 117.856) (width 0.7) (layer F.Cu) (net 1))
 (segment (start 126.619 119.888) (end 126.619 119.634) (width 0.7) (layer F.Cu) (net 1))
 (segment (start 130.175 116.085) (end 127.755 116.085) (width 0.7) (layer F.Cu) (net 1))
 (segment (start 122.421 116.99) (end 122.421 116.085) (width 0.7) (layer F.Cu) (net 1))
 (segment (start 125.319 119.888) (end 122.421 116.99) (width 0.7) (layer F.Cu) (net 1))
 (segment (start 126.619 119.888) (end 125.319 119.888) (width 0.7) (layer F.Cu) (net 1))
 (segment (start 122.421 116.085) (end 113.785 116.085) (width 0.7) (layer F.Cu) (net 1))
 (segment (start 127.755 116.085) (end 122.421 116.085) (width 0.7) (layer F.Cu) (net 1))
 (segment (start 130.429 116.339) (end 130.175 116.085) (width 0.7) (layer B.Cu) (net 1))
 (segment (start 130.429 118.244) (end 130.429 116.339) (width 0.7) (layer B.Cu) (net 1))
 (segment (start 148.717 112.776) (end 148.717 109.66401) (width 0.7) (layer B.Cu) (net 7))
 (segment (start 107.823 109.855) (end 113.85599 109.855) (width 0.7) (layer B.Cu) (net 7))
 (segment (start 100.584 112.772) (end 104.648 108.708) (width 0.7) (layer F.Cu) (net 18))
 (segment (start 104.648 108.708) (end 104.648 107.823) (width 0.7) (layer F.Cu) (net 18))
 (segment (start 105.156 107.315) (end 107.823 107.315) (width 0.7) (layer F.Cu) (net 18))
 (segment (start 104.648 107.823) (end 105.156 107.315) (width 0.7) (layer F.Cu) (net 18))
 (segment (start 107.823 107.315) (end 124.457194 107.315) (width 0.7) (layer F.Cu) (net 18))
 (segment (start 143.876989 115.076011) (end 146.177 112.776) (width 0.7) (layer F.Cu) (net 18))
 (segment (start 132.218205 115.076011) (end 143.876989 115.076011) (width 0.7) (layer F.Cu) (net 18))
 (segment (start 124.457194 107.315) (end 132.218205 115.076011) (width 0.7) (layer F.Cu) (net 18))
 (via (at 146.177 100.584) (size 1.2) (drill 0.6) (layers F.Cu B.Cu) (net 18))
 (segment (start 146.177 112.776) (end 146.177 100.584) (width 0.7) (layer F.Cu) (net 18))
 (via (at 141.859 100.584) (size 1.2) (drill 0.6) (layers F.Cu B.Cu) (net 18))
 (segment (start 146.177 100.584) (end 141.859 100.584) (width 0.7) (layer B.Cu) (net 18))
 (segment (start 141.859 100.584) (end 141.859 93.98) (width 0.7) (layer F.Cu) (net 18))
 (segment (start 141.859 93.98) (end 136.144 88.265) (width 0.7) (layer F.Cu) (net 18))
 (segment (start 136.144 85.09) (end 135.255 84.201) (width 0.7) (layer F.Cu) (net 18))
 (segment (start 136.144 88.265) (end 136.144 85.09) (width 0.7) (layer F.Cu) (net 18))
 (segment (start 100.584 110.482) (end 104.013 107.053) (width 0.7) (layer F.Cu) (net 11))
 (segment (start 104.013 107.053) (end 104.013 105.791) (width 0.7) (layer F.Cu) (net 11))
 (segment (start 105.029 104.775) (end 107.823 104.775) (width 0.7) (layer F.Cu) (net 11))
 (segment (start 104.013 105.791) (end 105.029 104.775) (width 0.7) (layer F.Cu) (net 11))
 (segment (start 107.823 104.775) (end 123.19 104.775) (width 0.7) (layer F.Cu) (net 11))
 (segment (start 142.236999 114.176001) (end 143.637 112.776) (width 0.7) (layer F.Cu) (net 11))
 (segment (start 132.591001 114.176001) (end 142.236999 114.176001) (width 0.7) (layer F.Cu) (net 11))
 (segment (start 123.19 104.775) (end 132.591001 114.176001) (width 0.7) (layer F.Cu) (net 11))
 (segment (start 143.637 94.742) (end 144.399 93.98) (width 0.7) (layer F.Cu) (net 11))
 (segment (start 143.637 112.776) (end 143.637 94.742) (width 0.7) (layer F.Cu) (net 11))
 (segment (start 144.399 93.98) (end 140.589 90.17) (width 0.7) (layer F.Cu) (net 11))
 (segment (start 140.589 84.455) (end 140.335 84.201) (width 0.7) (layer F.Cu) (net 11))
 (segment (start 140.589 90.17) (end 140.589 84.455) (width 0.7) (layer F.Cu) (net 11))
 (segment (start 136.779 93.98) (end 136.779 96.58399) (width 0.7) (layer B.Cu) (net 8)))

